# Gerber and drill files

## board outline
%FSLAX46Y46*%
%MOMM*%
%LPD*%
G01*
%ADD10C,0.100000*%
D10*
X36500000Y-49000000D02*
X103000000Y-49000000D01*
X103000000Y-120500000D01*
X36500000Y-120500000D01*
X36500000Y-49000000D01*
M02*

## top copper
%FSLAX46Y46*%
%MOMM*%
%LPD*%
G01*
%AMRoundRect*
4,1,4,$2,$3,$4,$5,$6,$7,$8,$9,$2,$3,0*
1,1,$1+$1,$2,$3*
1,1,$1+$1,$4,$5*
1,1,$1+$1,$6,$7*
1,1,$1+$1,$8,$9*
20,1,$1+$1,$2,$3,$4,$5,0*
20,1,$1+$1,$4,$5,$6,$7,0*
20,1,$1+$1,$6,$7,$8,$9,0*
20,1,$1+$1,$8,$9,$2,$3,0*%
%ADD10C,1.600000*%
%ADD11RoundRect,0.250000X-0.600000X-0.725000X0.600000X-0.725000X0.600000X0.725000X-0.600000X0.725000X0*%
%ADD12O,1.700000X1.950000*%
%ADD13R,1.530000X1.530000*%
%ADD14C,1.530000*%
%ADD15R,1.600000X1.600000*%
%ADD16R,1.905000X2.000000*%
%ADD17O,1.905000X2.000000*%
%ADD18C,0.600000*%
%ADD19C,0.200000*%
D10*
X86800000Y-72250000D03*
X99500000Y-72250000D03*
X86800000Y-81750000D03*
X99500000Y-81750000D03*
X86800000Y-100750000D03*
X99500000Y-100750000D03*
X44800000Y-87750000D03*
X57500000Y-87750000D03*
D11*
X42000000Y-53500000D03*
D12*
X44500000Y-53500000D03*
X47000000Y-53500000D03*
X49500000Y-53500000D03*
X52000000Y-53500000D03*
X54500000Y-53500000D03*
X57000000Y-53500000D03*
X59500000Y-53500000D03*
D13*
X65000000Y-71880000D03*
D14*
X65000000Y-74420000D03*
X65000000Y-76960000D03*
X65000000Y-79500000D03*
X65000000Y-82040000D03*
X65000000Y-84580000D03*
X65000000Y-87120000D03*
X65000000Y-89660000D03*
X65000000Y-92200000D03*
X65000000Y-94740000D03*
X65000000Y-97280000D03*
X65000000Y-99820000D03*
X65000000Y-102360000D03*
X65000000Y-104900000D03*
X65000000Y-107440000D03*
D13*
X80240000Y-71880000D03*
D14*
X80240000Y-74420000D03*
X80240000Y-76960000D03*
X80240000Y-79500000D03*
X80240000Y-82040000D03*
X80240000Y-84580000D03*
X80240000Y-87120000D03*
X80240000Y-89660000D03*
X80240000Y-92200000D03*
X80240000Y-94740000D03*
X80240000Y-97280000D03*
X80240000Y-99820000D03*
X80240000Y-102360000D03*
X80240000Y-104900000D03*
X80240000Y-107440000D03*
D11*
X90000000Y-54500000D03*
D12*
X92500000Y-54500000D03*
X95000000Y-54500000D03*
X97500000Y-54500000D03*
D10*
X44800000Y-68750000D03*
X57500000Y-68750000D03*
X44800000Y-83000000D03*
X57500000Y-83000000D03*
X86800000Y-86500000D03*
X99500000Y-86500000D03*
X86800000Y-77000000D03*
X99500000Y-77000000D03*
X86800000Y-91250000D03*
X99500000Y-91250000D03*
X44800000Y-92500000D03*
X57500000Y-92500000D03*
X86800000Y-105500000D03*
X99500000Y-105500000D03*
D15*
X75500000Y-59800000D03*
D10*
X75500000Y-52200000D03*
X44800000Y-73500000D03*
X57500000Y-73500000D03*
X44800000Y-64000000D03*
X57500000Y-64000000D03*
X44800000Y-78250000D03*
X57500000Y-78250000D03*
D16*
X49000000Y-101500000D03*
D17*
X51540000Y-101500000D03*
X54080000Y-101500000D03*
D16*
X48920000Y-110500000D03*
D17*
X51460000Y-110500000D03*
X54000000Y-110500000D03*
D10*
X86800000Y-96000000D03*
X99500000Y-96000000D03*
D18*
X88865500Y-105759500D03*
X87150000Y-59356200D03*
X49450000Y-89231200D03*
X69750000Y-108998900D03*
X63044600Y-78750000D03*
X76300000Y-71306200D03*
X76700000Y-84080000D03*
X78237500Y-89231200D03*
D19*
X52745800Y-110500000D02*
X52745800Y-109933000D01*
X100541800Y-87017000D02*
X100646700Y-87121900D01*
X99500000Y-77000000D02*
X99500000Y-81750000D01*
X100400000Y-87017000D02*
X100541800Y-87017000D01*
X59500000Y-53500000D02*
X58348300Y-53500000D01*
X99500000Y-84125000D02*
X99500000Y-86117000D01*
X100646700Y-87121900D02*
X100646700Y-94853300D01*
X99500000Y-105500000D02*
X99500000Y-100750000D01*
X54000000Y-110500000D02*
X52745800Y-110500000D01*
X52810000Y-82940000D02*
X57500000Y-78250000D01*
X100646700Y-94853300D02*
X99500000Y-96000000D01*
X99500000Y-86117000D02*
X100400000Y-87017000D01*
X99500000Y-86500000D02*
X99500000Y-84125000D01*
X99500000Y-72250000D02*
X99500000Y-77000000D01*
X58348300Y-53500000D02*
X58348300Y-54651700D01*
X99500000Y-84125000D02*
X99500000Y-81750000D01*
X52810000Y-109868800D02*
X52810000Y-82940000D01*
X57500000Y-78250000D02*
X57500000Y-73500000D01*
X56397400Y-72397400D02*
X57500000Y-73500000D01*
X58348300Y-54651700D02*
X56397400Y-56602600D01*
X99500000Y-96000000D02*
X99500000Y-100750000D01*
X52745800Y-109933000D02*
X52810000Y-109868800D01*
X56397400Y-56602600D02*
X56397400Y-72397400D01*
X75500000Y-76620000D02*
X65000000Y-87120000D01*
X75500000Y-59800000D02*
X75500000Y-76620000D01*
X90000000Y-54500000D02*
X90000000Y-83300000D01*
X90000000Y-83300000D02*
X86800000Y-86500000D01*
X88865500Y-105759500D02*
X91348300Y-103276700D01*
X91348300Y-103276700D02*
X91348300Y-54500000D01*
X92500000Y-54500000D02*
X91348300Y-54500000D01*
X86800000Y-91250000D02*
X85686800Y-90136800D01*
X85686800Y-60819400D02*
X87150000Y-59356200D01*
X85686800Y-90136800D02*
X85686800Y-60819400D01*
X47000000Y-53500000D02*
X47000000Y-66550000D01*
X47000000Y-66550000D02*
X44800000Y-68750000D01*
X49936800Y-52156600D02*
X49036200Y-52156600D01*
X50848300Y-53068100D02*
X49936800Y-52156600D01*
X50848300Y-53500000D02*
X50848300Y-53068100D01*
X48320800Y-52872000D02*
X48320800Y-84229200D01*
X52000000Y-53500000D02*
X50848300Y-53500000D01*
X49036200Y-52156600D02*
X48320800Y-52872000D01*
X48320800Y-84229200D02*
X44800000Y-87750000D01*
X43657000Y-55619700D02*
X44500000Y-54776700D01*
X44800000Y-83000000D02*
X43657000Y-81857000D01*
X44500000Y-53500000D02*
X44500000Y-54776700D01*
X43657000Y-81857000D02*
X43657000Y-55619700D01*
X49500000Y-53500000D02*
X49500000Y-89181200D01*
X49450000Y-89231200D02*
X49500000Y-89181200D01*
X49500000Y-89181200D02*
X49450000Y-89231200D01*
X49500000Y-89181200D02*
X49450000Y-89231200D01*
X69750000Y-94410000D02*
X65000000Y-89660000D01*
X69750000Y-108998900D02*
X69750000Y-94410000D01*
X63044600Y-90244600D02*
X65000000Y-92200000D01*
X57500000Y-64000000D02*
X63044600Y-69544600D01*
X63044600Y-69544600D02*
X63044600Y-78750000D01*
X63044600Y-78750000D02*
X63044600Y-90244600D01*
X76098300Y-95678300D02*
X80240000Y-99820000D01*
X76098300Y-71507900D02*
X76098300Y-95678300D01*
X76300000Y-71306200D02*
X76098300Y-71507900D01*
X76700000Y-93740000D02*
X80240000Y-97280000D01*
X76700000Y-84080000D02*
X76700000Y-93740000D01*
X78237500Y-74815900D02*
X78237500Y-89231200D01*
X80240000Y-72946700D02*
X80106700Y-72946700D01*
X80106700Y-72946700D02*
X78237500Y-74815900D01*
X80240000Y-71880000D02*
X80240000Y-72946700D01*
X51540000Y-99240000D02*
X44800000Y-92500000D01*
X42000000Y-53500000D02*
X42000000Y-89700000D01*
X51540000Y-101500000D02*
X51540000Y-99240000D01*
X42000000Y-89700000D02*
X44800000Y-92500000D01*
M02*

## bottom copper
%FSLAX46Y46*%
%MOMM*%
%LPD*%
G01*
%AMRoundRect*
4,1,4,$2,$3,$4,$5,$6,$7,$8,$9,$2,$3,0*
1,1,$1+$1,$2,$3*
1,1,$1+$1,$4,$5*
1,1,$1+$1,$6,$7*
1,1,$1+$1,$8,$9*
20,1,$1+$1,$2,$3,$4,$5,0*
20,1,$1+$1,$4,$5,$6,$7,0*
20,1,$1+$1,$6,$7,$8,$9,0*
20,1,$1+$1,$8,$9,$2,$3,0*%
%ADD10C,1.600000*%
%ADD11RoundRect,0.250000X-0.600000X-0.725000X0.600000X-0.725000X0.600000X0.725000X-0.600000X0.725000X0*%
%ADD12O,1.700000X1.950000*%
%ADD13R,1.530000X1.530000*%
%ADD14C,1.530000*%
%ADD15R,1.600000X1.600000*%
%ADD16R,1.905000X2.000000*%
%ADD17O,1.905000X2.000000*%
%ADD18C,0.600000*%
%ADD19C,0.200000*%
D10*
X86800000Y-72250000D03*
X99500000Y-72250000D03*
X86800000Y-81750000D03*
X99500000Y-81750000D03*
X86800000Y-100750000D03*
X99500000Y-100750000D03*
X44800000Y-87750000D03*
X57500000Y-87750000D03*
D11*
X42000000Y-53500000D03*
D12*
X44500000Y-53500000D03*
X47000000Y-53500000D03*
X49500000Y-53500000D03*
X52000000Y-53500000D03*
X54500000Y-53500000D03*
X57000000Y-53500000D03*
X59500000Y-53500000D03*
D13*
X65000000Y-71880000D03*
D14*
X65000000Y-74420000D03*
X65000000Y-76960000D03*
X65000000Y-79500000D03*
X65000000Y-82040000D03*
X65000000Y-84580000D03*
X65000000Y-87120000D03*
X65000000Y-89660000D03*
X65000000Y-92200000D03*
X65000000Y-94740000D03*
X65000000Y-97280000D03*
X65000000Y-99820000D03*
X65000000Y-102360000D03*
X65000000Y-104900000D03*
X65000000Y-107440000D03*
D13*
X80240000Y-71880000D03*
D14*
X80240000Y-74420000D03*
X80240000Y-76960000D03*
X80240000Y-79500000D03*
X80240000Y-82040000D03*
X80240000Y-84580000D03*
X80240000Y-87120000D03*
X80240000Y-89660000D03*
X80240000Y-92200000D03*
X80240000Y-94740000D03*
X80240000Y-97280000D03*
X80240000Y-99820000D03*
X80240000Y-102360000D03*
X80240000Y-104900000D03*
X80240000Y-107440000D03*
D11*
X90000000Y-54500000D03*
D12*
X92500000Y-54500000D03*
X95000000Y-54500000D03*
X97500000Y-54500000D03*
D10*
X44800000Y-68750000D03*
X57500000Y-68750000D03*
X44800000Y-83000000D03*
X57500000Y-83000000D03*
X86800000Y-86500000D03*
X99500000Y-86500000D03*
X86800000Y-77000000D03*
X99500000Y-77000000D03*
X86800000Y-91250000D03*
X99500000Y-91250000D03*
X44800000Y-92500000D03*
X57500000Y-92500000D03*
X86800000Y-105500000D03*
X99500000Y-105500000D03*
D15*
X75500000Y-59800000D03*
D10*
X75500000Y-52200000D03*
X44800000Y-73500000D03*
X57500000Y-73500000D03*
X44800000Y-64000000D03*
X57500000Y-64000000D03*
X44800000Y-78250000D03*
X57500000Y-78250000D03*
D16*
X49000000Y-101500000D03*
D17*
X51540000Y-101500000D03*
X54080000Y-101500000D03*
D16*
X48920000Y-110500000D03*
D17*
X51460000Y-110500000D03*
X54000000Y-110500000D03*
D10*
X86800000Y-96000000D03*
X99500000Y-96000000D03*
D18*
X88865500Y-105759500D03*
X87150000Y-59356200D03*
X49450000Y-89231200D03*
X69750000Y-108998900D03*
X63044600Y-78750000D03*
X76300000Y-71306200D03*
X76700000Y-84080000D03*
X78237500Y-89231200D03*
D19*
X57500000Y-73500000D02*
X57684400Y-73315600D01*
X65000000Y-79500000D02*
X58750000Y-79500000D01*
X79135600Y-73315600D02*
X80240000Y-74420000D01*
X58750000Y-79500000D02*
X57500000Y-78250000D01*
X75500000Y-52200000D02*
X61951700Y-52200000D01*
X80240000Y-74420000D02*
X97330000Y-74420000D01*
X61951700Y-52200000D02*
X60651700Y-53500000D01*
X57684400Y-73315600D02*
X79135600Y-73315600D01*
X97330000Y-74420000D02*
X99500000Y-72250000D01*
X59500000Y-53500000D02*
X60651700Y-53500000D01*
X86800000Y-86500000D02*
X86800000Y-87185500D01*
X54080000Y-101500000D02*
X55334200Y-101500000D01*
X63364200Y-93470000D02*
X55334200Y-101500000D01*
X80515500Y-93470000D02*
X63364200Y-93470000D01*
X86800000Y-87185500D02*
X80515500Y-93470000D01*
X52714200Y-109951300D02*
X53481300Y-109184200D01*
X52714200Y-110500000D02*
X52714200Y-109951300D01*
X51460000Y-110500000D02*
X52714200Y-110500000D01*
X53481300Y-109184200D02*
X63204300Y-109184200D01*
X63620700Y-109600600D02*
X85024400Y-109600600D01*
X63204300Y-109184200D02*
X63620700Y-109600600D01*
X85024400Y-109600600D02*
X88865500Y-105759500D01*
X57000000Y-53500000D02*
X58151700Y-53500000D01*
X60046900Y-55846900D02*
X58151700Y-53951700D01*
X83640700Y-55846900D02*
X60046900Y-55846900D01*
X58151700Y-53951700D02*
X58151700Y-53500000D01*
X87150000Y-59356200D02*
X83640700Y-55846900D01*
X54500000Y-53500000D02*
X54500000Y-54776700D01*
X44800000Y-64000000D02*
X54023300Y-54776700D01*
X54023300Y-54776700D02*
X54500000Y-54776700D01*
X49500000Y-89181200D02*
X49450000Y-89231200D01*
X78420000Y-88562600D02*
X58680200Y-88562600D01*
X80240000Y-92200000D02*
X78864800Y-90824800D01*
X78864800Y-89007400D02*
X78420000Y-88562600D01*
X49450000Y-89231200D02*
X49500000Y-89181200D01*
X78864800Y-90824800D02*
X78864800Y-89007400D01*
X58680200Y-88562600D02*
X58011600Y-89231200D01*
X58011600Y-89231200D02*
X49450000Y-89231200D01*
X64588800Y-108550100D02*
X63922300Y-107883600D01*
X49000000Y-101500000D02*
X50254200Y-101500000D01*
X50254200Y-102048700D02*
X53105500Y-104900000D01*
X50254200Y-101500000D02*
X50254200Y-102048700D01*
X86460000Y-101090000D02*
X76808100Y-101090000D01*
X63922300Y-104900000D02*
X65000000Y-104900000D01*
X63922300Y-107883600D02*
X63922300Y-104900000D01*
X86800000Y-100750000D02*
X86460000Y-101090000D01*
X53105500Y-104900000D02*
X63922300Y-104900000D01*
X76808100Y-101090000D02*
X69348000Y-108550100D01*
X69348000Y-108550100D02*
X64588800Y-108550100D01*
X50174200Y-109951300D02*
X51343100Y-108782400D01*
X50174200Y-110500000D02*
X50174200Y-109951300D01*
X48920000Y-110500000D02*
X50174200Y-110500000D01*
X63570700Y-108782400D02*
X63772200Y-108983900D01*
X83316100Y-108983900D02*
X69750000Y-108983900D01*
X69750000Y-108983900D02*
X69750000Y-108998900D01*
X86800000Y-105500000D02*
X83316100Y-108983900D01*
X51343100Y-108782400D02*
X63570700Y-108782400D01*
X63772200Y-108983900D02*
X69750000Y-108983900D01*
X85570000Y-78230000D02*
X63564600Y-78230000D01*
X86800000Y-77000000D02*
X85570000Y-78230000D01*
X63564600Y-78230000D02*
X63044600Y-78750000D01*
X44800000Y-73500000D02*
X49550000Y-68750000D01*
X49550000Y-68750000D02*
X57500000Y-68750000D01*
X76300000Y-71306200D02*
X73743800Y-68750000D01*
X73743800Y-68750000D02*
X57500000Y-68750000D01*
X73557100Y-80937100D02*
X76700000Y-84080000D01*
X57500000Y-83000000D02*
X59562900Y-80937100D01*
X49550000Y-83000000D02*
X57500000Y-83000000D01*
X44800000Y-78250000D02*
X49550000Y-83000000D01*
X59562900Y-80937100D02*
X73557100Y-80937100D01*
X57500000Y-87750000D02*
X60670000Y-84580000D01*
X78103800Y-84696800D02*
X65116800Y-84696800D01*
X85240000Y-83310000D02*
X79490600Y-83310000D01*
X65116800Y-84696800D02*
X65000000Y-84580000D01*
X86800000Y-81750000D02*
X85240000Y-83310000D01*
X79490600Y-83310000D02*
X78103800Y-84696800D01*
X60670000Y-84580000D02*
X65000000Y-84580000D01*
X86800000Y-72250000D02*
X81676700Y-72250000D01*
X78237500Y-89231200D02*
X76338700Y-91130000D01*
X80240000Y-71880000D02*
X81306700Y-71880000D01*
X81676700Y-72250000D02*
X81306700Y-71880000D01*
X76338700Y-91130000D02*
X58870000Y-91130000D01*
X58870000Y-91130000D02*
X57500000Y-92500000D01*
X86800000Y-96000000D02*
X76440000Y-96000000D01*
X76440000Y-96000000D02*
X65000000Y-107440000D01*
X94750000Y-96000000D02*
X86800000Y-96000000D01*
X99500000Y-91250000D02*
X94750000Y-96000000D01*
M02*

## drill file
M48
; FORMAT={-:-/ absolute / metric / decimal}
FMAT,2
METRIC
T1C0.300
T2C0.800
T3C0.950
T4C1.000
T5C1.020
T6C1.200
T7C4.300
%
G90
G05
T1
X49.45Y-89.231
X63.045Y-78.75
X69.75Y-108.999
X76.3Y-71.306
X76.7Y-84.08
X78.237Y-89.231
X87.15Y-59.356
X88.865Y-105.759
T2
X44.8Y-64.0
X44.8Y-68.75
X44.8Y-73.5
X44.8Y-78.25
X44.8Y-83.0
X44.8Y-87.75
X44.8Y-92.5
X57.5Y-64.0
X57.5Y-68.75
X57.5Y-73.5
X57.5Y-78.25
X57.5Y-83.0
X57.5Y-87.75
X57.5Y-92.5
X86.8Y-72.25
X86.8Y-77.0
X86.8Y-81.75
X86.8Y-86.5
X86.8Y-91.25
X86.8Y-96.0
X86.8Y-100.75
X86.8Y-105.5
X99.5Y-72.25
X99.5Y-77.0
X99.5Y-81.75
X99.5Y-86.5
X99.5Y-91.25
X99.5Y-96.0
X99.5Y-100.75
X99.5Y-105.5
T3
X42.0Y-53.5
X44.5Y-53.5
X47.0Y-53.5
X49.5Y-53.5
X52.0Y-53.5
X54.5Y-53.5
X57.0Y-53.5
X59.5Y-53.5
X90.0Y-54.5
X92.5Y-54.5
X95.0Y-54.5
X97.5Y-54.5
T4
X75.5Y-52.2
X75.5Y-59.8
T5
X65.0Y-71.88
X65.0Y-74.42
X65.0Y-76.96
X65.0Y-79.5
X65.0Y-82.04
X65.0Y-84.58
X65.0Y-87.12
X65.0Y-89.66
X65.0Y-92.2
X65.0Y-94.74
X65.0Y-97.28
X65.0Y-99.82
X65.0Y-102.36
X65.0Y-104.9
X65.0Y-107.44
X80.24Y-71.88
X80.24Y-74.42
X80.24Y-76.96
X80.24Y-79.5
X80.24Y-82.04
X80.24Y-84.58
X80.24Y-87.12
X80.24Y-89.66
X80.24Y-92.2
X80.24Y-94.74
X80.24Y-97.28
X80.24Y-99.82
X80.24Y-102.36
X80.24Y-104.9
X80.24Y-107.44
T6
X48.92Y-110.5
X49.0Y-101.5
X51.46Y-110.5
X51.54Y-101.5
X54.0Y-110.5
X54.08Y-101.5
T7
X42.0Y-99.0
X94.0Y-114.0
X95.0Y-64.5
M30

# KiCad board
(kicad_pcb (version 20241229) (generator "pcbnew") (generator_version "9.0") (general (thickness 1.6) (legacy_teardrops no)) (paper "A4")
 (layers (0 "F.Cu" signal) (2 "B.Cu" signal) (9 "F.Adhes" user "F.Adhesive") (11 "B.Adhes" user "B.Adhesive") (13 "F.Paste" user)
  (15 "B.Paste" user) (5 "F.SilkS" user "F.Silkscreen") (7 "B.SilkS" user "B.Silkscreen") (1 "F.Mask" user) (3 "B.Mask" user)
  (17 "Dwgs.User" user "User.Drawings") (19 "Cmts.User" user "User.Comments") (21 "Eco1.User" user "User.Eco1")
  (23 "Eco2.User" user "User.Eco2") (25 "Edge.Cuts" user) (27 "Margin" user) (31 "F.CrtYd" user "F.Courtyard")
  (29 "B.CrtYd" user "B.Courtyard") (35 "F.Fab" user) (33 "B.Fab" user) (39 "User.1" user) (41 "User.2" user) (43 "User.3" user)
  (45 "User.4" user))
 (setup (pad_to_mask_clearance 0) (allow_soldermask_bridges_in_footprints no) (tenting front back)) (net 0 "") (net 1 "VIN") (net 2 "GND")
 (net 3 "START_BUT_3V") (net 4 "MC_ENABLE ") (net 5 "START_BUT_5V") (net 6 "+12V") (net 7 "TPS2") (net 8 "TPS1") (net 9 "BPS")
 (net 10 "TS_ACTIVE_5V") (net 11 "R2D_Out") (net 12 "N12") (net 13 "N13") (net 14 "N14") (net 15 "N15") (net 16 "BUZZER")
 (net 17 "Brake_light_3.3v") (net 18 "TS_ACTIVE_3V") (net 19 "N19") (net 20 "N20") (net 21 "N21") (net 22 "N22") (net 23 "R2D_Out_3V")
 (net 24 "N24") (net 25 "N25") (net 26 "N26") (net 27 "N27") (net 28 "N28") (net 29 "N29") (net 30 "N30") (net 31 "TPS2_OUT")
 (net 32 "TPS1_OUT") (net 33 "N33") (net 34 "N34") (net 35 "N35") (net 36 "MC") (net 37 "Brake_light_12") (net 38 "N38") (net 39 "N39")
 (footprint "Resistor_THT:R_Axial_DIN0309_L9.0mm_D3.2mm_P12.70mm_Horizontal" (layer "F.Cu") (at 86.8 72.25)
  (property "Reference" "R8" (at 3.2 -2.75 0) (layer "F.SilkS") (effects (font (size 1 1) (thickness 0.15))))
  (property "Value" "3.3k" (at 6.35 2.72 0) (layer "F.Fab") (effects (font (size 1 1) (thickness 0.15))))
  (pad "1" thru_hole circle (at 0 0) (size 1.6 1.6) (drill 0.8) (layers "*.Cu" "*.Mask") (remove_unused_layers no) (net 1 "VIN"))
  (pad "2" thru_hole circle (at 12.7 0) (size 1.6 1.6) (drill 0.8) (layers "*.Cu" "*.Mask") (remove_unused_layers no) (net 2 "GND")))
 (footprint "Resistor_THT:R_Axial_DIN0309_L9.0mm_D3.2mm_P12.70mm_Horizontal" (layer "F.Cu") (at 86.8 81.75)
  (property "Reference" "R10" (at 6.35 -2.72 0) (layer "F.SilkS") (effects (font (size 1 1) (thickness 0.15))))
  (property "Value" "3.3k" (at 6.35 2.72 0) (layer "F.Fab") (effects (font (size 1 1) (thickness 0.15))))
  (pad "1" thru_hole circle (at 0 0) (size 1.6 1.6) (drill 0.8) (layers "*.Cu" "*.Mask") (remove_unused_layers no) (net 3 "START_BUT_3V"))
  (pad "2" thru_hole circle (at 12.7 0) (size 1.6 1.6) (drill 0.8) (layers "*.Cu" "*.Mask") (remove_unused_layers no) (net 2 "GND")))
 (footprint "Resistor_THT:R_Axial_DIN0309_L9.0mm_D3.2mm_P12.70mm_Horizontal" (layer "F.Cu") (at 86.8 100.75)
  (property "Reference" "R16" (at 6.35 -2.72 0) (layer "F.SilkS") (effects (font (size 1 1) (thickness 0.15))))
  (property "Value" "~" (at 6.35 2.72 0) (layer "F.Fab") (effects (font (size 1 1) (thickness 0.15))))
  (pad "1" thru_hole circle (at 0 0) (size 1.6 1.6) (drill 0.8) (layers "*.Cu" "*.Mask") (remove_unused_layers no) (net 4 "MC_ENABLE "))
  (pad "2" thru_hole circle (at 12.7 0) (size 1.6 1.6) (drill 0.8) (layers "*.Cu" "*.Mask") (remove_unused_layers no) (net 2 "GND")))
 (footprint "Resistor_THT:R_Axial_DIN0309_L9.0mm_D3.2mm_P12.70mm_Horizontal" (layer "F.Cu") (at 44.8 87.75)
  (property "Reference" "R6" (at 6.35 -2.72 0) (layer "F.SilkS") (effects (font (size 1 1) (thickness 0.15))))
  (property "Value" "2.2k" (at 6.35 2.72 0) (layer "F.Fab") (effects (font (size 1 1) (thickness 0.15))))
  (pad "1" thru_hole circle (at 0 0) (size 1.6 1.6) (drill 0.8) (layers "*.Cu" "*.Mask") (remove_unused_layers no) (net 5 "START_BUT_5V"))
  (pad "2" thru_hole circle (at 12.7 0) (size 1.6 1.6) (drill 0.8) (layers "*.Cu" "*.Mask") (remove_unused_layers no) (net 3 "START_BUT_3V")))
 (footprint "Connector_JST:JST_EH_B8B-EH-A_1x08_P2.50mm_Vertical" (layer "F.Cu") (at 42 53.5)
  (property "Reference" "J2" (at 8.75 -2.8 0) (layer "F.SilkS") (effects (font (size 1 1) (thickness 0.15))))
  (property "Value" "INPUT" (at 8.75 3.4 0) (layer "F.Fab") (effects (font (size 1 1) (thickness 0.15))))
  (pad "1" thru_hole roundrect (at 0 0) (size 1.7 1.95) (drill 0.95) (layers "*.Cu" "*.Mask") (remove_unused_layers no)
   (roundrect_rratio 0.147059) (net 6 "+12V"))
  (pad "2" thru_hole oval (at 2.5 0) (size 1.7 1.95) (drill 0.95) (layers "*.Cu" "*.Mask") (remove_unused_layers no) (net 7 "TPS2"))
  (pad "3" thru_hole oval (at 5 0) (size 1.7 1.95) (drill 0.95) (layers "*.Cu" "*.Mask") (remove_unused_layers no) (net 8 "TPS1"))
  (pad "4" thru_hole oval (at 7.5 0) (size 1.7 1.95) (drill 0.95) (layers "*.Cu" "*.Mask") (remove_unused_layers no) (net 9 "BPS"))
  (pad "5" thru_hole oval (at 10 0) (size 1.7 1.95) (drill 0.95) (layers "*.Cu" "*.Mask") (remove_unused_layers no) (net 5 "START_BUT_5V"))
  (pad "6" thru_hole oval (at 12.5 0) (size 1.7 1.95) (drill 0.95) (layers "*.Cu" "*.Mask") (remove_unused_layers no)
   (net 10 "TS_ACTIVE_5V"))
  (pad "7" thru_hole oval (at 15 0) (size 1.7 1.95) (drill 0.95) (layers "*.Cu" "*.Mask") (remove_unused_layers no) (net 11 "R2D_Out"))
  (pad "8" thru_hole oval (at 17.5 0) (size 1.7 1.95) (drill 0.95) (layers "*.Cu" "*.Mask") (remove_unused_layers no) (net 2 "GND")))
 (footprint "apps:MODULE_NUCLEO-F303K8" (layer "F.Cu") (at 72.62 89.66)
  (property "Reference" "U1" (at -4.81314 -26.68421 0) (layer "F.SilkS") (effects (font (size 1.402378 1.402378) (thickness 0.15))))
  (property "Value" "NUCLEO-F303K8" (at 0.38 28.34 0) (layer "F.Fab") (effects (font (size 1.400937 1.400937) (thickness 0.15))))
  (pad "3_1" thru_hole rect (at -7.62 -17.78) (size 1.53 1.53) (drill 1.02) (layers "*.Cu" "*.Mask") (remove_unused_layers no)
   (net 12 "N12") (solder_mask_margin 0.102))
  (pad "3_2" thru_hole circle (at -7.62 -15.24) (size 1.53 1.53) (drill 1.02) (layers "*.Cu" "*.Mask") (remove_unused_layers no)
   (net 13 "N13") (solder_mask_margin 0.102))
  (pad "3_3" thru_hole circle (at -7.62 -12.7) (size 1.53 1.53) (drill 1.02) (layers "*.Cu" "*.Mask") (remove_unused_layers no)
   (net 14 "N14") (solder_mask_margin 0.102))
  (pad "3_4" thru_hole circle (at -7.62 -10.16) (size 1.53 1.53) (drill 1.02) (layers "*.Cu" "*.Mask") (remove_unused_layers no)
   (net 2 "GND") (solder_mask_margin 0.102))
  (pad "3_5" thru_hole circle (at -7.62 -7.62) (size 1.53 1.53) (drill 1.02) (layers "*.Cu" "*.Mask") (remove_unused_layers no)
   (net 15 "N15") (solder_mask_margin 0.102))
  (pad "3_6" thru_hole circle (at -7.62 -5.08) (size 1.53 1.53) (drill 1.02) (layers "*.Cu" "*.Mask") (remove_unused_layers no)
   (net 3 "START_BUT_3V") (solder_mask_margin 0.102))
  (pad "3_7" thru_hole circle (at -7.62 -2.54) (size 1.53 1.53) (drill 1.02) (layers "*.Cu" "*.Mask") (remove_unused_layers no)
   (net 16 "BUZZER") (solder_mask_margin 0.102))
  (pad "3_8" thru_hole circle (at -7.62 0) (size 1.53 1.53) (drill 1.02) (layers "*.Cu" "*.Mask") (remove_unused_layers no)
   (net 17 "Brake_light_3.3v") (solder_mask_margin 0.102))
  (pad "3_9" thru_hole circle (at -7.62 2.54) (size 1.53 1.53) (drill 1.02) (layers "*.Cu" "*.Mask") (remove_unused_layers no)
   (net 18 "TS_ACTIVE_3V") (solder_mask_margin 0.102))
  (pad "3_10" thru_hole circle (at -7.62 5.08) (size 1.53 1.53) (drill 1.02) (layers "*.Cu" "*.Mask") (remove_unused_layers no)
   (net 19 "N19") (solder_mask_margin 0.102))
  (pad "3_11" thru_hole circle (at -7.62 7.62) (size 1.53 1.53) (drill 1.02) (layers "*.Cu" "*.Mask") (remove_unused_layers no)
   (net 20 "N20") (solder_mask_margin 0.102))
  (pad "3_12" thru_hole circle (at -7.62 10.16) (size 1.53 1.53) (drill 1.02) (layers "*.Cu" "*.Mask") (remove_unused_layers no)
   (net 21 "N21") (solder_mask_margin 0.102))
  (pad "3_13" thru_hole circle (at -7.62 12.7) (size 1.53 1.53) (drill 1.02) (layers "*.Cu" "*.Mask") (remove_unused_layers no)
   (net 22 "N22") (solder_mask_margin 0.102))
  (pad "3_14" thru_hole circle (at -7.62 15.24) (size 1.53 1.53) (drill 1.02) (layers "*.Cu" "*.Mask") (remove_unused_layers no)
   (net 4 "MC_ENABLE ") (solder_mask_margin 0.102))
  (pad "3_15" thru_hole circle (at -7.62 17.78) (size 1.53 1.53) (drill 1.02) (layers "*.Cu" "*.Mask") (remove_unused_layers no)
   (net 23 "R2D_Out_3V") (solder_mask_margin 0.102))
  (pad "4_1" thru_hole rect (at 7.62 -17.78) (size 1.53 1.53) (drill 1.02) (layers "*.Cu" "*.Mask") (remove_unused_layers no) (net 1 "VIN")
   (solder_mask_margin 0.102))
  (pad "4_2" thru_hole circle (at 7.62 -15.24) (size 1.53 1.53) (drill 1.02) (layers "*.Cu" "*.Mask") (remove_unused_layers no)
   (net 2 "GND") (solder_mask_margin 0.102))
  (pad "4_3" thru_hole circle (at 7.62 -12.7) (size 1.53 1.53) (drill 1.02) (layers "*.Cu" "*.Mask") (remove_unused_layers no)
   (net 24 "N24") (solder_mask_margin 0.102))
  (pad "4_4" thru_hole circle (at 7.62 -10.16) (size 1.53 1.53) (drill 1.02) (layers "*.Cu" "*.Mask") (remove_unused_layers no)
   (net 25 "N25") (solder_mask_margin 0.102))
  (pad "4_5" thru_hole circle (at 7.62 -7.62) (size 1.53 1.53) (drill 1.02) (layers "*.Cu" "*.Mask") (remove_unused_layers no)
   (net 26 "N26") (solder_mask_margin 0.102))
  (pad "4_6" thru_hole circle (at 7.62 -5.08) (size 1.53 1.53) (drill 1.02) (layers "*.Cu" "*.Mask") (remove_unused_layers no)
   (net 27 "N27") (solder_mask_margin 0.102))
  (pad "4_7" thru_hole circle (at 7.62 -2.54) (size 1.53 1.53) (drill 1.02) (layers "*.Cu" "*.Mask") (remove_unused_layers no)
   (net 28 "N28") (solder_mask_margin 0.102))
  (pad "4_8" thru_hole circle (at 7.62 0) (size 1.53 1.53) (drill 1.02) (layers "*.Cu" "*.Mask") (remove_unused_layers no) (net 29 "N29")
   (solder_mask_margin 0.102))
  (pad "4_9" thru_hole circle (at 7.62 2.54) (size 1.53 1.53) (drill 1.02) (layers "*.Cu" "*.Mask") (remove_unused_layers no) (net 9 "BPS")
   (solder_mask_margin 0.102))
  (pad "4_10" thru_hole circle (at 7.62 5.08) (size 1.53 1.53) (drill 1.02) (layers "*.Cu" "*.Mask") (remove_unused_layers no)
   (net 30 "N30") (solder_mask_margin 0.102))
  (pad "4_11" thru_hole circle (at 7.62 7.62) (size 1.53 1.53) (drill 1.02) (layers "*.Cu" "*.Mask") (remove_unused_layers no)
   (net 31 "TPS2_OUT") (solder_mask_margin 0.102))
  (pad "4_12" thru_hole circle (at 7.62 10.16) (size 1.53 1.53) (drill 1.02) (layers "*.Cu" "*.Mask") (remove_unused_layers no)
   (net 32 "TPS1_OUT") (solder_mask_margin 0.102))
  (pad "4_13" thru_hole circle (at 7.62 12.7) (size 1.53 1.53) (drill 1.02) (layers "*.Cu" "*.Mask") (remove_unused_layers no)
   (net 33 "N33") (solder_mask_margin 0.102))
  (pad "4_14" thru_hole circle (at 7.62 15.24) (size 1.53 1.53) (drill 1.02) (layers "*.Cu" "*.Mask") (remove_unused_layers no)
   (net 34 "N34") (solder_mask_margin 0.102))
  (pad "4_15" thru_hole circle (at 7.62 17.78) (size 1.53 1.53) (drill 1.02) (layers "*.Cu" "*.Mask") (remove_unused_layers no)
   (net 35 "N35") (solder_mask_margin 0.102)))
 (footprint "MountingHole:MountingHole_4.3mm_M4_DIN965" (layer "F.Cu") (at 94 114)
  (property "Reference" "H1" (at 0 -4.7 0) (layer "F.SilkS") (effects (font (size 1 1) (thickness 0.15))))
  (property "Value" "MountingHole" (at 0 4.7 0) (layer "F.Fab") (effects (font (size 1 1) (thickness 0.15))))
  (pad "" np_thru_hole circle (at 0 0) (size 4.3 4.3) (drill 4.3) (layers "*.Cu" "*.Mask")))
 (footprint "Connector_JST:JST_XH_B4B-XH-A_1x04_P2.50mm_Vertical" (layer "F.Cu") (at 90 54.5)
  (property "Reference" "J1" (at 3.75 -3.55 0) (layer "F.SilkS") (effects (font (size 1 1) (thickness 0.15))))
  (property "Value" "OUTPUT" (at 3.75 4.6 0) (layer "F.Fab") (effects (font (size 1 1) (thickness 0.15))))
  (pad "1" thru_hole roundrect (at 0 0) (size 1.7 1.95) (drill 0.95) (layers "*.Cu" "*.Mask") (remove_unused_layers no)
   (roundrect_rratio 0.147059) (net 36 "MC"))
  (pad "2" thru_hole oval (at 2.5 0) (size 1.7 1.95) (drill 0.95) (layers "*.Cu" "*.Mask") (remove_unused_layers no)
   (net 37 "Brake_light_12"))
  (pad "3" thru_hole oval (at 5 0) (size 1.7 1.95) (drill 0.95) (layers "*.Cu" "*.Mask") (remove_unused_layers no) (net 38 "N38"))
  (pad "4" thru_hole oval (at 7.5 0) (size 1.7 1.95) (drill 0.95) (layers "*.Cu" "*.Mask") (remove_unused_layers no) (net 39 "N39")))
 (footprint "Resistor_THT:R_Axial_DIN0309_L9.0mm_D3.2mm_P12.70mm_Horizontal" (layer "F.Cu") (at 44.8 68.75)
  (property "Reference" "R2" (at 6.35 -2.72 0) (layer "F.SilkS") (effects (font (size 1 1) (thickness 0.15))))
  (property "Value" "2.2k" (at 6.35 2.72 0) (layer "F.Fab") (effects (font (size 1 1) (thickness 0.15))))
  (pad "1" thru_hole circle (at 0 0) (size 1.6 1.6) (drill 0.8) (layers "*.Cu" "*.Mask") (remove_unused_layers no) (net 8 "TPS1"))
  (pad "2" thru_hole circle (at 12.7 0) (size 1.6 1.6) (drill 0.8) (layers "*.Cu" "*.Mask") (remove_unused_layers no) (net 32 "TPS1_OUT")))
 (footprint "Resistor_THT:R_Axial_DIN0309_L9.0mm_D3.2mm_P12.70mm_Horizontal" (layer "F.Cu") (at 44.8 83)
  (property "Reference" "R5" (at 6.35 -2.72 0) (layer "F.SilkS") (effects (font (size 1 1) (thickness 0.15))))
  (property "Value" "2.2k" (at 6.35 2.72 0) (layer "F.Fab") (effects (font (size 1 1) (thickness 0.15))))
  (pad "1" thru_hole circle (at 0 0) (size 1.6 1.6) (drill 0.8) (layers "*.Cu" "*.Mask") (remove_unused_layers no) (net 7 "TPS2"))
  (pad "2" thru_hole circle (at 12.7 0) (size 1.6 1.6) (drill 0.8) (layers "*.Cu" "*.Mask") (remove_unused_layers no) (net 31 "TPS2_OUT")))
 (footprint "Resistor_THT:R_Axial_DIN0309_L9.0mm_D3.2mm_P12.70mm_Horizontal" (layer "F.Cu") (at 86.8 86.5)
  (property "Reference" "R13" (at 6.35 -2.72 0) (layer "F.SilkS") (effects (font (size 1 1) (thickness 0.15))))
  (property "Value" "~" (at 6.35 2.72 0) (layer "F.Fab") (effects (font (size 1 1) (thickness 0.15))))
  (pad "1" thru_hole circle (at 0 0) (size 1.6 1.6) (drill 0.8) (layers "*.Cu" "*.Mask") (remove_unused_layers no) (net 36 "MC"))
  (pad "2" thru_hole circle (at 12.7 0) (size 1.6 1.6) (drill 0.8) (layers "*.Cu" "*.Mask") (remove_unused_layers no) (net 2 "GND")))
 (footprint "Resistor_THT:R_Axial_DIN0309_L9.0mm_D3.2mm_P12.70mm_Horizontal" (layer "F.Cu") (at 86.8 77)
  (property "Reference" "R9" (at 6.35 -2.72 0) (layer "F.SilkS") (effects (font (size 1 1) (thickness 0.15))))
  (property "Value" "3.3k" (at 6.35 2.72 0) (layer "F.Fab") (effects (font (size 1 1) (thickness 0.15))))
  (pad "1" thru_hole circle (at 0 0) (size 1.6 1.6) (drill 0.8) (layers "*.Cu" "*.Mask") (remove_unused_layers no) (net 18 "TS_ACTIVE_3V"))
  (pad "2" thru_hole circle (at 12.7 0) (size 1.6 1.6) (drill 0.8) (layers "*.Cu" "*.Mask") (remove_unused_layers no) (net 2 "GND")))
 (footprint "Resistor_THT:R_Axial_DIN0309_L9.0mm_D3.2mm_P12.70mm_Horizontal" (layer "F.Cu") (at 86.8 91.25)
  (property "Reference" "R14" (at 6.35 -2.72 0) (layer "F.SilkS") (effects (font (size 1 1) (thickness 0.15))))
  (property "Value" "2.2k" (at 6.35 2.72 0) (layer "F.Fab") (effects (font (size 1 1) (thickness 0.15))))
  (pad "1" thru_hole circle (at 0 0) (size 1.6 1.6) (drill 0.8) (layers "*.Cu" "*.Mask") (remove_unused_layers no) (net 11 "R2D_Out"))
  (pad "2" thru_hole circle (at 12.7 0) (size 1.6 1.6) (drill 0.8) (layers "*.Cu" "*.Mask") (remove_unused_layers no) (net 23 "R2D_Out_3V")))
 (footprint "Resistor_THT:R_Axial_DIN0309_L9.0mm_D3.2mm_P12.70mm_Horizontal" (layer "F.Cu") (at 44.8 92.5)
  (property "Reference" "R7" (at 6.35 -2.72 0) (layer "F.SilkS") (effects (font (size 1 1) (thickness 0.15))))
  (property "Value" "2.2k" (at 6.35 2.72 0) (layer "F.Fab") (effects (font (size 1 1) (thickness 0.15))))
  (pad "1" thru_hole circle (at 0 0) (size 1.6 1.6) (drill 0.8) (layers "*.Cu" "*.Mask") (remove_unused_layers no) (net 6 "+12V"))
  (pad "2" thru_hole circle (at 12.7 0) (size 1.6 1.6) (drill 0.8) (layers "*.Cu" "*.Mask") (remove_unused_layers no) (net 1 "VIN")))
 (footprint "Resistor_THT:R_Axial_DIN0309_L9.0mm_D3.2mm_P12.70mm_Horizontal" (layer "F.Cu") (at 86.8 105.5)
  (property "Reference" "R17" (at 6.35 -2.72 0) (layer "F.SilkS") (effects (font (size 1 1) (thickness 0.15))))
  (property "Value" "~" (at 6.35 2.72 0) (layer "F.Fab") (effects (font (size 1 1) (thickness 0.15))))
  (pad "1" thru_hole circle (at 0 0) (size 1.6 1.6) (drill 0.8) (layers "*.Cu" "*.Mask") (remove_unused_layers no)
   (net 17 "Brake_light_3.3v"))
  (pad "2" thru_hole circle (at 12.7 0) (size 1.6 1.6) (drill 0.8) (layers "*.Cu" "*.Mask") (remove_unused_layers no) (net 2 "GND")))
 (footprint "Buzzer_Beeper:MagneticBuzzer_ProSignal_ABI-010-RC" (layer "F.Cu") (at 75.5 59.8 90)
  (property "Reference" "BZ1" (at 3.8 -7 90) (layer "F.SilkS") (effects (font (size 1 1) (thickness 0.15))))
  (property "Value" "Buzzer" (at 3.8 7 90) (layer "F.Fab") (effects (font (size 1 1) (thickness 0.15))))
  (pad "1" thru_hole rect (at 0 0 90) (size 1.6 1.6) (drill 1) (layers "*.Cu" "*.Mask") (remove_unused_layers no) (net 16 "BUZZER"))
  (pad "2" thru_hole circle (at 7.6 0 90) (size 1.6 1.6) (drill 1) (layers "*.Cu" "*.Mask") (remove_unused_layers no) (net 2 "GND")))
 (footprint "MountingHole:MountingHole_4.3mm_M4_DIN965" (layer "F.Cu") (at 95 64.5 90)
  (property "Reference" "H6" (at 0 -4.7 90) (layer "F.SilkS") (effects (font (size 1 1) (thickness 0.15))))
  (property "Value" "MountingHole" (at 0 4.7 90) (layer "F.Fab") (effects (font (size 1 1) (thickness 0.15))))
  (pad "" np_thru_hole circle (at 0 0 90) (size 4.3 4.3) (drill 4.3) (layers "*.Cu" "*.Mask")))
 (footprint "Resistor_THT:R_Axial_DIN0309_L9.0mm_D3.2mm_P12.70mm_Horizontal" (layer "F.Cu") (at 44.8 73.5)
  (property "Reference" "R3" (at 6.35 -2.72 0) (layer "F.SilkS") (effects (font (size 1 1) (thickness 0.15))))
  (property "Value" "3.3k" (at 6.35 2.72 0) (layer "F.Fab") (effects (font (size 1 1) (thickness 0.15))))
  (pad "1" thru_hole circle (at 0 0) (size 1.6 1.6) (drill 0.8) (layers "*.Cu" "*.Mask") (remove_unused_layers no) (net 32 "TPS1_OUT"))
  (pad "2" thru_hole circle (at 12.7 0) (size 1.6 1.6) (drill 0.8) (layers "*.Cu" "*.Mask") (remove_unused_layers no) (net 2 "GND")))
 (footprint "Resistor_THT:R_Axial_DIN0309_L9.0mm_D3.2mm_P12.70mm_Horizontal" (layer "F.Cu") (at 44.8 64)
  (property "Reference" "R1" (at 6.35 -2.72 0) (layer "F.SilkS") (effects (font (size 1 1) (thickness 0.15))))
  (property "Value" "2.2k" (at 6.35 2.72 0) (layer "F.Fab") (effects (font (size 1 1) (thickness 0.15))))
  (pad "1" thru_hole circle (at 0 0) (size 1.6 1.6) (drill 0.8) (layers "*.Cu" "*.Mask") (remove_unused_layers no) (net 10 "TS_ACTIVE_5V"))
  (pad "2" thru_hole circle (at 12.7 0) (size 1.6 1.6) (drill 0.8) (layers "*.Cu" "*.Mask") (remove_unused_layers no)
   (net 18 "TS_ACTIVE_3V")))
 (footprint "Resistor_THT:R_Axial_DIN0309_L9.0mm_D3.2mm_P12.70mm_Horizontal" (layer "F.Cu") (at 44.8 78.25)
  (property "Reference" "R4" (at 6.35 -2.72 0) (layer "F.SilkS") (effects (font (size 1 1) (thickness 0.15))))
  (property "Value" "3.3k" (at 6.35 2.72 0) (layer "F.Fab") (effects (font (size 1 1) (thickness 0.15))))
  (pad "1" thru_hole circle (at 0 0) (size 1.6 1.6) (drill 0.8) (layers "*.Cu" "*.Mask") (remove_unused_layers no) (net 31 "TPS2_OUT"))
  (pad "2" thru_hole circle (at 12.7 0) (size 1.6 1.6) (drill 0.8) (layers "*.Cu" "*.Mask") (remove_unused_layers no) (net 2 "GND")))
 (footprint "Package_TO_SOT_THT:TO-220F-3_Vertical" (layer "F.Cu") (at 49 101.5)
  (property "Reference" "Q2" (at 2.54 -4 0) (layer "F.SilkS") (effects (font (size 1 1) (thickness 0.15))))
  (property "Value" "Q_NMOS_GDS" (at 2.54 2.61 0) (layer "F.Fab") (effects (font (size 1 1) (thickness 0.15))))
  (pad "1" thru_hole rect (at 0 0) (size 1.905 2) (drill 1.2) (layers "*.Cu" "*.Mask") (remove_unused_layers no) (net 4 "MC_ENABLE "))
  (pad "2" thru_hole oval (at 2.54 0) (size 1.905 2) (drill 1.2) (layers "*.Cu" "*.Mask") (remove_unused_layers no) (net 6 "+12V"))
  (pad "3" thru_hole oval (at 5.08 0) (size 1.905 2) (drill 1.2) (layers "*.Cu" "*.Mask") (remove_unused_layers no) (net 36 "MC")))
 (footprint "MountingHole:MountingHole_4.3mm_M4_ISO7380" (layer "F.Cu") (at 42 99)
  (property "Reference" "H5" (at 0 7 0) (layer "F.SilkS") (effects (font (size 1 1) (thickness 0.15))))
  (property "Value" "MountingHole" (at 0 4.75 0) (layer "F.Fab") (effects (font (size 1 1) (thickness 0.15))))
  (pad "" np_thru_hole circle (at 0 0) (size 4.3 4.3) (drill 4.3) (layers "*.Cu" "*.Mask")))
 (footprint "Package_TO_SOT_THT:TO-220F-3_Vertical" (layer "F.Cu") (at 48.92 110.5)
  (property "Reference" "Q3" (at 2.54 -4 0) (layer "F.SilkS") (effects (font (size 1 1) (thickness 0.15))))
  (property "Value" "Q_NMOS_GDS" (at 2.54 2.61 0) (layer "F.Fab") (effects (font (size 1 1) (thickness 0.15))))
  (pad "1" thru_hole rect (at 0 0) (size 1.905 2) (drill 1.2) (layers "*.Cu" "*.Mask") (remove_unused_layers no) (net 17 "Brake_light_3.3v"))
  (pad "2" thru_hole oval (at 2.54 0) (size 1.905 2) (drill 1.2) (layers "*.Cu" "*.Mask") (remove_unused_layers no)
   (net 37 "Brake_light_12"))
  (pad "3" thru_hole oval (at 5.08 0) (size 1.905 2) (drill 1.2) (layers "*.Cu" "*.Mask") (remove_unused_layers no) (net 2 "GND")))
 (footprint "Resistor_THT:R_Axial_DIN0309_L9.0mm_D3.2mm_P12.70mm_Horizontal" (layer "F.Cu") (at 86.8 96)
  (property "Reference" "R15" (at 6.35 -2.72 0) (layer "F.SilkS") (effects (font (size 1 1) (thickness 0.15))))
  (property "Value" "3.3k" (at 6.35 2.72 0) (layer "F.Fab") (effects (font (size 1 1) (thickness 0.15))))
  (pad "1" thru_hole circle (at 0 0) (size 1.6 1.6) (drill 0.8) (layers "*.Cu" "*.Mask") (remove_unused_layers no) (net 23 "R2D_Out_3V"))
  (pad "2" thru_hole circle (at 12.7 0) (size 1.6 1.6) (drill 0.8) (layers "*.Cu" "*.Mask") (remove_unused_layers no) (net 2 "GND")))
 (gr_rect (start 36.5 49) (end 103 120.5) (stroke (width 0.1) (type solid)) (fill no) (layer "Edge.Cuts"))
 (segment (start 52.7458 110.5) (end 52.7458 109.933) (width 0.2) (layer "F.Cu") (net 2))
 (segment (start 100.5418 87.017) (end 100.6467 87.1219) (width 0.2) (layer "F.Cu") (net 2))
 (segment (start 99.5 77) (end 99.5 81.75) (width 0.2) (layer "F.Cu") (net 2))
 (segment (start 100.4 87.017) (end 100.5418 87.017) (width 0.2) (layer "F.Cu") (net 2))
 (segment (start 59.5 53.5) (end 58.3483 53.5) (width 0.2) (layer "F.Cu") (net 2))
 (segment (start 99.5 84.125) (end 99.5 86.117) (width 0.2) (layer "F.Cu") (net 2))
 (segment (start 100.6467 87.1219) (end 100.6467 94.8533) (width 0.2) (layer "F.Cu") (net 2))
 (segment (start 99.5 105.5) (end 99.5 100.75) (width 0.2) (layer "F.Cu") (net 2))
 (segment (start 54 110.5) (end 52.7458 110.5) (width 0.2) (layer "F.Cu") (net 2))
 (segment (start 52.81 82.94) (end 57.5 78.25) (width 0.2) (layer "F.Cu") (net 2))
 (segment (start 100.6467 94.8533) (end 99.5 96) (width 0.2) (layer "F.Cu") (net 2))
 (segment (start 99.5 86.117) (end 100.4 87.017) (width 0.2) (layer "F.Cu") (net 2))
 (segment (start 99.5 86.5) (end 99.5 84.125) (width 0.2) (layer "F.Cu") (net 2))
 (segment (start 99.5 72.25) (end 99.5 77) (width 0.2) (layer "F.Cu") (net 2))
 (segment (start 58.3483 53.5) (end 58.3483 54.6517) (width 0.2) (layer "F.Cu") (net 2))
 (segment (start 99.5 84.125) (end 99.5 81.75) (width 0.2) (layer "F.Cu") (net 2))
 (segment (start 52.81 109.8688) (end 52.81 82.94) (width 0.2) (layer "F.Cu") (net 2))
 (segment (start 57.5 78.25) (end 57.5 73.5) (width 0.2) (layer "F.Cu") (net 2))
 (segment (start 56.3974 72.3974) (end 57.5 73.5) (width 0.2) (layer "F.Cu") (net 2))
 (segment (start 58.3483 54.6517) (end 56.3974 56.6026) (width 0.2) (layer "F.Cu") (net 2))
 (segment (start 99.5 96) (end 99.5 100.75) (width 0.2) (layer "F.Cu") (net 2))
 (segment (start 52.7458 109.933) (end 52.81 109.8688) (width 0.2) (layer "F.Cu") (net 2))
 (segment (start 56.3974 56.6026) (end 56.3974 72.3974) (width 0.2) (layer "F.Cu") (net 2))
 (segment (start 57.5 73.5) (end 57.6844 73.3156) (width 0.2) (layer "B.Cu") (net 2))
 (segment (start 65 79.5) (end 58.75 79.5) (width 0.2) (layer "B.Cu") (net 2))
 (segment (start 79.1356 73.3156) (end 80.24 74.42) (width 0.2) (layer "B.Cu") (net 2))
 (segment (start 58.75 79.5) (end 57.5 78.25) (width 0.2) (layer "B.Cu") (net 2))
 (segment (start 75.5 52.2) (end 61.9517 52.2) (width 0.2) (layer "B.Cu") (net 2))
 (segment (start 80.24 74.42) (end 97.33 74.42) (width 0.2) (layer "B.Cu") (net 2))
 (segment (start 61.9517 52.2) (end 60.6517 53.5) (width 0.2) (layer "B.Cu") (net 2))
 (segment (start 57.6844 73.3156) (end 79.1356 73.3156) (width 0.2) (layer "B.Cu") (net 2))
 (segment (start 97.33 74.42) (end 99.5 72.25) (width 0.2) (layer "B.Cu") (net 2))
 (segment (start 59.5 53.5) (end 60.6517 53.5) (width 0.2) (layer "B.Cu") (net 2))
 (segment (start 75.5 76.62) (end 65 87.12) (width 0.2) (layer "F.Cu") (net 16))
 (segment (start 75.5 59.8) (end 75.5 76.62) (width 0.2) (layer "F.Cu") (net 16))
 (segment (start 90 54.5) (end 90 83.3) (width 0.2) (layer "F.Cu") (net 36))
 (segment (start 90 83.3) (end 86.8 86.5) (width 0.2) (layer "F.Cu") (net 36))
 (segment (start 86.8 86.5) (end 86.8 87.1855) (width 0.2) (layer "B.Cu") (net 36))
 (segment (start 54.08 101.5) (end 55.3342 101.5) (width 0.2) (layer "B.Cu") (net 36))
 (segment (start 63.3642 93.47) (end 55.3342 101.5) (width 0.2) (layer "B.Cu") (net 36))
 (segment (start 80.5155 93.47) (end 63.3642 93.47) (width 0.2) (layer "B.Cu") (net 36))
 (segment (start 86.8 87.1855) (end 80.5155 93.47) (width 0.2) (layer "B.Cu") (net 36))
 (segment (start 88.8655 105.7595) (end 91.3483 103.2767) (width 0.2) (layer "F.Cu") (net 37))
 (segment (start 91.3483 103.2767) (end 91.3483 54.5) (width 0.2) (layer "F.Cu") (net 37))
 (segment (start 92.5 54.5) (end 91.3483 54.5) (width 0.2) (layer "F.Cu") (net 37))
 (via (at 88.8655 105.7595) (size 0.6) (drill 0.3) (layers "F.Cu" "B.Cu") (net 37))
 (segment (start 52.7142 109.9513) (end 53.4813 109.1842) (width 0.2) (layer "B.Cu") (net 37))
 (segment (start 52.7142 110.5) (end 52.7142 109.9513) (width 0.2) (layer "B.Cu") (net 37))
 (segment (start 51.46 110.5) (end 52.7142 110.5) (width 0.2) (layer "B.Cu") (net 37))
 (segment (start 53.4813 109.1842) (end 63.2043 109.1842) (width 0.2) (layer "B.Cu") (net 37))
 (segment (start 63.6207 109.6006) (end 85.0244 109.6006) (width 0.2) (layer "B.Cu") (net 37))
 (segment (start 63.2043 109.1842) (end 63.6207 109.6006) (width 0.2) (layer "B.Cu") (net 37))
 (segment (start 85.0244 109.6006) (end 88.8655 105.7595) (width 0.2) (layer "B.Cu") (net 37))
 (segment (start 86.8 91.25) (end 85.6868 90.1368) (width 0.2) (layer "F.Cu") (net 11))
 (segment (start 85.6868 60.8194) (end 87.15 59.3562) (width 0.2) (layer "F.Cu") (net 11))
 (segment (start 85.6868 90.1368) (end 85.6868 60.8194) (width 0.2) (layer "F.Cu") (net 11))
 (via (at 87.15 59.3562) (size 0.6) (drill 0.3) (layers "F.Cu" "B.Cu") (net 11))
 (segment (start 57 53.5) (end 58.1517 53.5) (width 0.2) (layer "B.Cu") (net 11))
 (segment (start 60.0469 55.8469) (end 58.1517 53.9517) (width 0.2) (layer "B.Cu") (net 11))
 (segment (start 83.6407 55.8469) (end 60.0469 55.8469) (width 0.2) (layer "B.Cu") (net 11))
 (segment (start 58.1517 53.9517) (end 58.1517 53.5) (width 0.2) (layer "B.Cu") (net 11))
 (segment (start 87.15 59.3562) (end 83.6407 55.8469) (width 0.2) (layer "B.Cu") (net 11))
 (segment (start 47 53.5) (end 47 66.55) (width 0.2) (layer "F.Cu") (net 8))
 (segment (start 47 66.55) (end 44.8 68.75) (width 0.2) (layer "F.Cu") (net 8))
 (segment (start 54.5 53.5) (end 54.5 54.7767) (width 0.2) (layer "B.Cu") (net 10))
 (segment (start 44.8 64) (end 54.0233 54.7767) (width 0.2) (layer "B.Cu") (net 10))
 (segment (start 54.0233 54.7767) (end 54.5 54.7767) (width 0.2) (layer "B.Cu") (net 10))
 (segment (start 49.9368 52.1566) (end 49.0362 52.1566) (width 0.2) (layer "F.Cu") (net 5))
 (segment (start 50.8483 53.0681) (end 49.9368 52.1566) (width 0.2) (layer "F.Cu") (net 5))
 (segment (start 50.8483 53.5) (end 50.8483 53.0681) (width 0.2) (layer "F.Cu") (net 5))
 (segment (start 48.3208 52.872) (end 48.3208 84.2292) (width 0.2) (layer "F.Cu") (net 5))
 (segment (start 52 53.5) (end 50.8483 53.5) (width 0.2) (layer "F.Cu") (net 5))
 (segment (start 49.0362 52.1566) (end 48.3208 52.872) (width 0.2) (layer "F.Cu") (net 5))
 (segment (start 48.3208 84.2292) (end 44.8 87.75) (width 0.2) (layer "F.Cu") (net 5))
 (segment (start 43.657 55.6197) (end 44.5 54.7767) (width 0.2) (layer "F.Cu") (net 7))
 (segment (start 44.8 83) (end 43.657 81.857) (width 0.2) (layer "F.Cu") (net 7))
 (segment (start 44.5 53.5) (end 44.5 54.7767) (width 0.2) (layer "F.Cu") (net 7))
 (segment (start 43.657 81.857) (end 43.657 55.6197) (width 0.2) (layer "F.Cu") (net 7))
 (segment (start 49.5 53.5) (end 49.5 89.1812) (width 0.2) (layer "F.Cu") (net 9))
 (segment (start 49.45 89.2312) (end 49.5 89.1812) (width 0.2) (layer "F.Cu") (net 9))
 (segment (start 49.5 89.1812) (end 49.45 89.2312) (width 0.2) (layer "F.Cu") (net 9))
 (segment (start 49.5 89.1812) (end 49.45 89.2312) (width 0.2) (layer "F.Cu") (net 9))
 (via (at 49.45 89.2312) (size 0.6) (drill 0.3) (layers "F.Cu" "B.Cu") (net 9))
 (segment (start 49.5 89.1812) (end 49.45 89.2312) (width 0.2) (layer "B.Cu") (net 9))
 (segment (start 78.42 88.5626) (end 58.6802 88.5626) (width 0.2) (layer "B.Cu") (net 9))
 (segment (start 80.24 92.2) (end 78.8648 90.8248) (width 0.2) (layer "B.Cu") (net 9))
 (segment (start 78.8648 89.0074) (end 78.42 88.5626) (width 0.2) (layer "B.Cu") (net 9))
 (segment (start 49.45 89.2312) (end 49.5 89.1812) (width 0.2) (layer "B.Cu") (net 9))
 (segment (start 78.8648 90.8248) (end 78.8648 89.0074) (width 0.2) (layer "B.Cu") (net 9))
 (segment (start 58.6802 88.5626) (end 58.0116 89.2312) (width 0.2) (layer "B.Cu") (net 9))
 (segment (start 58.0116 89.2312) (end 49.45 89.2312) (width 0.2) (layer "B.Cu") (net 9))
 (segment (start 64.5888 108.5501) (end 63.9223 107.8836) (width 0.2) (layer "B.Cu") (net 4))
 (segment (start 49 101.5) (end 50.2542 101.5) (width 0.2) (layer "B.Cu") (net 4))
 (segment (start 50.2542 102.0487) (end 53.1055 104.9) (width 0.2) (layer "B.Cu") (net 4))
 (segment (start 50.2542 101.5) (end 50.2542 102.0487) (width 0.2) (layer "B.Cu") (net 4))
 (segment (start 86.46 101.09) (end 76.8081 101.09) (width 0.2) (layer "B.Cu") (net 4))
 (segment (start 63.9223 104.9) (end 65 104.9) (width 0.2) (layer "B.Cu") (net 4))
 (segment (start 63.9223 107.8836) (end 63.9223 104.9) (width 0.2) (layer "B.Cu") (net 4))
 (segment (start 86.8 100.75) (end 86.46 101.09) (width 0.2) (layer "B.Cu") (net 4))
 (segment (start 53.1055 104.9) (end 63.9223 104.9) (width 0.2) (layer "B.Cu") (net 4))
 (segment (start 76.8081 101.09) (end 69.348 108.5501) (width 0.2) (layer "B.Cu") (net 4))
 (segment (start 69.348 108.5501) (end 64.5888 108.5501) (width 0.2) (layer "B.Cu") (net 4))
 (segment (start 69.75 94.41) (end 65 89.66) (width 0.2) (layer "F.Cu") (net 17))
 (segment (start 69.75 108.9989) (end 69.75 94.41) (width 0.2) (layer "F.Cu") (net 17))
 (via (at 69.75 108.9989) (size 0.6) (drill 0.3) (layers "F.Cu" "B.Cu") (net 17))
 (segment (start 50.1742 109.9513) (end 51.3431 108.7824) (width 0.2) (layer "B.Cu") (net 17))
 (segment (start 50.1742 110.5) (end 50.1742 109.9513) (width 0.2) (layer "B.Cu") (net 17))
 (segment (start 48.92 110.5) (end 50.1742 110.5) (width 0.2) (layer "B.Cu") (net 17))
 (segment (start 63.5707 108.7824) (end 63.7722 108.9839) (width 0.2) (layer "B.Cu") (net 17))
 (segment (start 83.3161 108.9839) (end 69.75 108.9839) (width 0.2) (layer "B.Cu") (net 17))
 (segment (start 69.75 108.9839) (end 69.75 108.9989) (width 0.2) (layer "B.Cu") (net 17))
 (segment (start 86.8 105.5) (end 83.3161 108.9839) (width 0.2) (layer "B.Cu") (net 17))
 (segment (start 51.3431 108.7824) (end 63.5707 108.7824) (width 0.2) (layer "B.Cu") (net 17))
 (segment (start 63.7722 108.9839) (end 69.75 108.9839) (width 0.2) (layer "B.Cu") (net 17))
 (segment (start 63.0446 90.2446) (end 65 92.2) (width 0.2) (layer "F.Cu") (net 18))
 (segment (start 57.5 64) (end 63.0446 69.5446) (width 0.2) (layer "F.Cu") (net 18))
 (segment (start 63.0446 69.5446) (end 63.0446 78.75) (width 0.2) (layer "F.Cu") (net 18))
 (segment (start 63.0446 78.75) (end 63.0446 90.2446) (width 0.2) (layer "F.Cu") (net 18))
 (via (at 63.0446 78.75) (size 0.6) (drill 0.3) (layers "F.Cu" "B.Cu") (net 18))
 (segment (start 85.57 78.23) (end 63.5646 78.23) (width 0.2) (layer "B.Cu") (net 18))
 (segment (start 86.8 77) (end 85.57 78.23) (width 0.2) (layer "B.Cu") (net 18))
 (segment (start 63.5646 78.23) (end 63.0446 78.75) (width 0.2) (layer "B.Cu") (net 18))
 (segment (start 76.0983 95.6783) (end 80.24 99.82) (width 0.2) (layer "F.Cu") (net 32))
 (segment (start 76.0983 71.5079) (end 76.0983 95.6783) (width 0.2) (layer "F.Cu") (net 32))
 (segment (start 76.3 71.3062) (end 76.0983 71.5079) (width 0.2) (layer "F.Cu") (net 32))
 (via (at 76.3 71.3062) (size 0.6) (drill 0.3) (layers "F.Cu" "B.Cu") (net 32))
 (segment (start 44.8 73.5) (end 49.55 68.75) (width 0.2) (layer "B.Cu") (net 32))
 (segment (start 49.55 68.75) (end 57.5 68.75) (width 0.2) (layer "B.Cu") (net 32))
 (segment (start 76.3 71.3062) (end 73.7438 68.75) (width 0.2) (layer "B.Cu") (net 32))
 (segment (start 73.7438 68.75) (end 57.5 68.75) (width 0.2) (layer "B.Cu") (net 32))
 (segment (start 76.7 93.74) (end 80.24 97.28) (width 0.2) (layer "F.Cu") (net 31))
 (segment (start 76.7 84.08) (end 76.7 93.74) (width 0.2) (layer "F.Cu") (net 31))
 (via (at 76.7 84.08) (size 0.6) (drill 0.3) (layers "F.Cu" "B.Cu") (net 31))
 (segment (start 73.5571 80.9371) (end 76.7 84.08) (width 0.2) (layer "B.Cu") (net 31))
 (segment (start 57.5 83) (end 59.5629 80.9371) (width 0.2) (layer "B.Cu") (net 31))
 (segment (start 49.55 83) (end 57.5 83) (width 0.2) (layer "B.Cu") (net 31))
 (segment (start 44.8 78.25) (end 49.55 83) (width 0.2) (layer "B.Cu") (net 31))
 (segment (start 59.5629 80.9371) (end 73.5571 80.9371) (width 0.2) (layer "B.Cu") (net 31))
 (segment (start 57.5 87.75) (end 60.67 84.58) (width 0.2) (layer "B.Cu") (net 3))
 (segment (start 78.1038 84.6968) (end 65.1168 84.6968) (width 0.2) (layer "B.Cu") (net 3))
 (segment (start 85.24 83.31) (end 79.4906 83.31) (width 0.2) (layer "B.Cu") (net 3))
 (segment (start 65.1168 84.6968) (end 65 84.58) (width 0.2) (layer "B.Cu") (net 3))
 (segment (start 86.8 81.75) (end 85.24 83.31) (width 0.2) (layer "B.Cu") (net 3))
 (segment (start 79.4906 83.31) (end 78.1038 84.6968) (width 0.2) (layer "B.Cu") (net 3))
 (segment (start 60.67 84.58) (end 65 84.58) (width 0.2) (layer "B.Cu") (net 3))
 (segment (start 78.2375 74.8159) (end 78.2375 89.2312) (width 0.2) (layer "F.Cu") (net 1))
 (segment (start 80.24 72.9467) (end 80.1067 72.9467) (width 0.2) (layer "F.Cu") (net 1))
 (segment (start 80.1067 72.9467) (end 78.2375 74.8159) (width 0.2) (layer "F.Cu") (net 1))
 (segment (start 80.24 71.88) (end 80.24 72.9467) (width 0.2) (layer "F.Cu") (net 1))
 (via (at 78.2375 89.2312) (size 0.6) (drill 0.3) (layers "F.Cu" "B.Cu") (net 1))
 (segment (start 86.8 72.25) (end 81.6767 72.25) (width 0.2) (layer "B.Cu") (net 1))
 (segment (start 78.2375 89.2312) (end 76.3387 91.13) (width 0.2) (layer "B.Cu") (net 1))
 (segment (start 80.24 71.88) (end 81.3067 71.88) (width 0.2) (layer "B.Cu") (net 1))
 (segment (start 81.6767 72.25) (end 81.3067 71.88) (width 0.2) (layer "B.Cu") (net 1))
 (segment (start 76.3387 91.13) (end 58.87 91.13) (width 0.2) (layer "B.Cu") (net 1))
 (segment (start 58.87 91.13) (end 57.5 92.5) (width 0.2) (layer "B.Cu") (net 1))
 (segment (start 86.8 96) (end 76.44 96) (width 0.2) (layer "B.Cu") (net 23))
 (segment (start 76.44 96) (end 65 107.44) (width 0.2) (layer "B.Cu") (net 23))
 (segment (start 94.75 96) (end 86.8 96) (width 0.2) (layer "B.Cu") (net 23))
 (segment (start 99.5 91.25) (end 94.75 96) (width 0.2) (layer "B.Cu") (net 23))
 (segment (start 51.54 99.24) (end 44.8 92.5) (width 0.2) (layer "F.Cu") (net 6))
 (segment (start 42 53.5) (end 42 89.7) (width 0.2) (layer "F.Cu") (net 6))
 (segment (start 51.54 101.5) (end 51.54 99.24) (width 0.2) (layer "F.Cu") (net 6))
 (segment (start 42 89.7) (end 44.8 92.5) (width 0.2) (layer "F.Cu") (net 6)))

